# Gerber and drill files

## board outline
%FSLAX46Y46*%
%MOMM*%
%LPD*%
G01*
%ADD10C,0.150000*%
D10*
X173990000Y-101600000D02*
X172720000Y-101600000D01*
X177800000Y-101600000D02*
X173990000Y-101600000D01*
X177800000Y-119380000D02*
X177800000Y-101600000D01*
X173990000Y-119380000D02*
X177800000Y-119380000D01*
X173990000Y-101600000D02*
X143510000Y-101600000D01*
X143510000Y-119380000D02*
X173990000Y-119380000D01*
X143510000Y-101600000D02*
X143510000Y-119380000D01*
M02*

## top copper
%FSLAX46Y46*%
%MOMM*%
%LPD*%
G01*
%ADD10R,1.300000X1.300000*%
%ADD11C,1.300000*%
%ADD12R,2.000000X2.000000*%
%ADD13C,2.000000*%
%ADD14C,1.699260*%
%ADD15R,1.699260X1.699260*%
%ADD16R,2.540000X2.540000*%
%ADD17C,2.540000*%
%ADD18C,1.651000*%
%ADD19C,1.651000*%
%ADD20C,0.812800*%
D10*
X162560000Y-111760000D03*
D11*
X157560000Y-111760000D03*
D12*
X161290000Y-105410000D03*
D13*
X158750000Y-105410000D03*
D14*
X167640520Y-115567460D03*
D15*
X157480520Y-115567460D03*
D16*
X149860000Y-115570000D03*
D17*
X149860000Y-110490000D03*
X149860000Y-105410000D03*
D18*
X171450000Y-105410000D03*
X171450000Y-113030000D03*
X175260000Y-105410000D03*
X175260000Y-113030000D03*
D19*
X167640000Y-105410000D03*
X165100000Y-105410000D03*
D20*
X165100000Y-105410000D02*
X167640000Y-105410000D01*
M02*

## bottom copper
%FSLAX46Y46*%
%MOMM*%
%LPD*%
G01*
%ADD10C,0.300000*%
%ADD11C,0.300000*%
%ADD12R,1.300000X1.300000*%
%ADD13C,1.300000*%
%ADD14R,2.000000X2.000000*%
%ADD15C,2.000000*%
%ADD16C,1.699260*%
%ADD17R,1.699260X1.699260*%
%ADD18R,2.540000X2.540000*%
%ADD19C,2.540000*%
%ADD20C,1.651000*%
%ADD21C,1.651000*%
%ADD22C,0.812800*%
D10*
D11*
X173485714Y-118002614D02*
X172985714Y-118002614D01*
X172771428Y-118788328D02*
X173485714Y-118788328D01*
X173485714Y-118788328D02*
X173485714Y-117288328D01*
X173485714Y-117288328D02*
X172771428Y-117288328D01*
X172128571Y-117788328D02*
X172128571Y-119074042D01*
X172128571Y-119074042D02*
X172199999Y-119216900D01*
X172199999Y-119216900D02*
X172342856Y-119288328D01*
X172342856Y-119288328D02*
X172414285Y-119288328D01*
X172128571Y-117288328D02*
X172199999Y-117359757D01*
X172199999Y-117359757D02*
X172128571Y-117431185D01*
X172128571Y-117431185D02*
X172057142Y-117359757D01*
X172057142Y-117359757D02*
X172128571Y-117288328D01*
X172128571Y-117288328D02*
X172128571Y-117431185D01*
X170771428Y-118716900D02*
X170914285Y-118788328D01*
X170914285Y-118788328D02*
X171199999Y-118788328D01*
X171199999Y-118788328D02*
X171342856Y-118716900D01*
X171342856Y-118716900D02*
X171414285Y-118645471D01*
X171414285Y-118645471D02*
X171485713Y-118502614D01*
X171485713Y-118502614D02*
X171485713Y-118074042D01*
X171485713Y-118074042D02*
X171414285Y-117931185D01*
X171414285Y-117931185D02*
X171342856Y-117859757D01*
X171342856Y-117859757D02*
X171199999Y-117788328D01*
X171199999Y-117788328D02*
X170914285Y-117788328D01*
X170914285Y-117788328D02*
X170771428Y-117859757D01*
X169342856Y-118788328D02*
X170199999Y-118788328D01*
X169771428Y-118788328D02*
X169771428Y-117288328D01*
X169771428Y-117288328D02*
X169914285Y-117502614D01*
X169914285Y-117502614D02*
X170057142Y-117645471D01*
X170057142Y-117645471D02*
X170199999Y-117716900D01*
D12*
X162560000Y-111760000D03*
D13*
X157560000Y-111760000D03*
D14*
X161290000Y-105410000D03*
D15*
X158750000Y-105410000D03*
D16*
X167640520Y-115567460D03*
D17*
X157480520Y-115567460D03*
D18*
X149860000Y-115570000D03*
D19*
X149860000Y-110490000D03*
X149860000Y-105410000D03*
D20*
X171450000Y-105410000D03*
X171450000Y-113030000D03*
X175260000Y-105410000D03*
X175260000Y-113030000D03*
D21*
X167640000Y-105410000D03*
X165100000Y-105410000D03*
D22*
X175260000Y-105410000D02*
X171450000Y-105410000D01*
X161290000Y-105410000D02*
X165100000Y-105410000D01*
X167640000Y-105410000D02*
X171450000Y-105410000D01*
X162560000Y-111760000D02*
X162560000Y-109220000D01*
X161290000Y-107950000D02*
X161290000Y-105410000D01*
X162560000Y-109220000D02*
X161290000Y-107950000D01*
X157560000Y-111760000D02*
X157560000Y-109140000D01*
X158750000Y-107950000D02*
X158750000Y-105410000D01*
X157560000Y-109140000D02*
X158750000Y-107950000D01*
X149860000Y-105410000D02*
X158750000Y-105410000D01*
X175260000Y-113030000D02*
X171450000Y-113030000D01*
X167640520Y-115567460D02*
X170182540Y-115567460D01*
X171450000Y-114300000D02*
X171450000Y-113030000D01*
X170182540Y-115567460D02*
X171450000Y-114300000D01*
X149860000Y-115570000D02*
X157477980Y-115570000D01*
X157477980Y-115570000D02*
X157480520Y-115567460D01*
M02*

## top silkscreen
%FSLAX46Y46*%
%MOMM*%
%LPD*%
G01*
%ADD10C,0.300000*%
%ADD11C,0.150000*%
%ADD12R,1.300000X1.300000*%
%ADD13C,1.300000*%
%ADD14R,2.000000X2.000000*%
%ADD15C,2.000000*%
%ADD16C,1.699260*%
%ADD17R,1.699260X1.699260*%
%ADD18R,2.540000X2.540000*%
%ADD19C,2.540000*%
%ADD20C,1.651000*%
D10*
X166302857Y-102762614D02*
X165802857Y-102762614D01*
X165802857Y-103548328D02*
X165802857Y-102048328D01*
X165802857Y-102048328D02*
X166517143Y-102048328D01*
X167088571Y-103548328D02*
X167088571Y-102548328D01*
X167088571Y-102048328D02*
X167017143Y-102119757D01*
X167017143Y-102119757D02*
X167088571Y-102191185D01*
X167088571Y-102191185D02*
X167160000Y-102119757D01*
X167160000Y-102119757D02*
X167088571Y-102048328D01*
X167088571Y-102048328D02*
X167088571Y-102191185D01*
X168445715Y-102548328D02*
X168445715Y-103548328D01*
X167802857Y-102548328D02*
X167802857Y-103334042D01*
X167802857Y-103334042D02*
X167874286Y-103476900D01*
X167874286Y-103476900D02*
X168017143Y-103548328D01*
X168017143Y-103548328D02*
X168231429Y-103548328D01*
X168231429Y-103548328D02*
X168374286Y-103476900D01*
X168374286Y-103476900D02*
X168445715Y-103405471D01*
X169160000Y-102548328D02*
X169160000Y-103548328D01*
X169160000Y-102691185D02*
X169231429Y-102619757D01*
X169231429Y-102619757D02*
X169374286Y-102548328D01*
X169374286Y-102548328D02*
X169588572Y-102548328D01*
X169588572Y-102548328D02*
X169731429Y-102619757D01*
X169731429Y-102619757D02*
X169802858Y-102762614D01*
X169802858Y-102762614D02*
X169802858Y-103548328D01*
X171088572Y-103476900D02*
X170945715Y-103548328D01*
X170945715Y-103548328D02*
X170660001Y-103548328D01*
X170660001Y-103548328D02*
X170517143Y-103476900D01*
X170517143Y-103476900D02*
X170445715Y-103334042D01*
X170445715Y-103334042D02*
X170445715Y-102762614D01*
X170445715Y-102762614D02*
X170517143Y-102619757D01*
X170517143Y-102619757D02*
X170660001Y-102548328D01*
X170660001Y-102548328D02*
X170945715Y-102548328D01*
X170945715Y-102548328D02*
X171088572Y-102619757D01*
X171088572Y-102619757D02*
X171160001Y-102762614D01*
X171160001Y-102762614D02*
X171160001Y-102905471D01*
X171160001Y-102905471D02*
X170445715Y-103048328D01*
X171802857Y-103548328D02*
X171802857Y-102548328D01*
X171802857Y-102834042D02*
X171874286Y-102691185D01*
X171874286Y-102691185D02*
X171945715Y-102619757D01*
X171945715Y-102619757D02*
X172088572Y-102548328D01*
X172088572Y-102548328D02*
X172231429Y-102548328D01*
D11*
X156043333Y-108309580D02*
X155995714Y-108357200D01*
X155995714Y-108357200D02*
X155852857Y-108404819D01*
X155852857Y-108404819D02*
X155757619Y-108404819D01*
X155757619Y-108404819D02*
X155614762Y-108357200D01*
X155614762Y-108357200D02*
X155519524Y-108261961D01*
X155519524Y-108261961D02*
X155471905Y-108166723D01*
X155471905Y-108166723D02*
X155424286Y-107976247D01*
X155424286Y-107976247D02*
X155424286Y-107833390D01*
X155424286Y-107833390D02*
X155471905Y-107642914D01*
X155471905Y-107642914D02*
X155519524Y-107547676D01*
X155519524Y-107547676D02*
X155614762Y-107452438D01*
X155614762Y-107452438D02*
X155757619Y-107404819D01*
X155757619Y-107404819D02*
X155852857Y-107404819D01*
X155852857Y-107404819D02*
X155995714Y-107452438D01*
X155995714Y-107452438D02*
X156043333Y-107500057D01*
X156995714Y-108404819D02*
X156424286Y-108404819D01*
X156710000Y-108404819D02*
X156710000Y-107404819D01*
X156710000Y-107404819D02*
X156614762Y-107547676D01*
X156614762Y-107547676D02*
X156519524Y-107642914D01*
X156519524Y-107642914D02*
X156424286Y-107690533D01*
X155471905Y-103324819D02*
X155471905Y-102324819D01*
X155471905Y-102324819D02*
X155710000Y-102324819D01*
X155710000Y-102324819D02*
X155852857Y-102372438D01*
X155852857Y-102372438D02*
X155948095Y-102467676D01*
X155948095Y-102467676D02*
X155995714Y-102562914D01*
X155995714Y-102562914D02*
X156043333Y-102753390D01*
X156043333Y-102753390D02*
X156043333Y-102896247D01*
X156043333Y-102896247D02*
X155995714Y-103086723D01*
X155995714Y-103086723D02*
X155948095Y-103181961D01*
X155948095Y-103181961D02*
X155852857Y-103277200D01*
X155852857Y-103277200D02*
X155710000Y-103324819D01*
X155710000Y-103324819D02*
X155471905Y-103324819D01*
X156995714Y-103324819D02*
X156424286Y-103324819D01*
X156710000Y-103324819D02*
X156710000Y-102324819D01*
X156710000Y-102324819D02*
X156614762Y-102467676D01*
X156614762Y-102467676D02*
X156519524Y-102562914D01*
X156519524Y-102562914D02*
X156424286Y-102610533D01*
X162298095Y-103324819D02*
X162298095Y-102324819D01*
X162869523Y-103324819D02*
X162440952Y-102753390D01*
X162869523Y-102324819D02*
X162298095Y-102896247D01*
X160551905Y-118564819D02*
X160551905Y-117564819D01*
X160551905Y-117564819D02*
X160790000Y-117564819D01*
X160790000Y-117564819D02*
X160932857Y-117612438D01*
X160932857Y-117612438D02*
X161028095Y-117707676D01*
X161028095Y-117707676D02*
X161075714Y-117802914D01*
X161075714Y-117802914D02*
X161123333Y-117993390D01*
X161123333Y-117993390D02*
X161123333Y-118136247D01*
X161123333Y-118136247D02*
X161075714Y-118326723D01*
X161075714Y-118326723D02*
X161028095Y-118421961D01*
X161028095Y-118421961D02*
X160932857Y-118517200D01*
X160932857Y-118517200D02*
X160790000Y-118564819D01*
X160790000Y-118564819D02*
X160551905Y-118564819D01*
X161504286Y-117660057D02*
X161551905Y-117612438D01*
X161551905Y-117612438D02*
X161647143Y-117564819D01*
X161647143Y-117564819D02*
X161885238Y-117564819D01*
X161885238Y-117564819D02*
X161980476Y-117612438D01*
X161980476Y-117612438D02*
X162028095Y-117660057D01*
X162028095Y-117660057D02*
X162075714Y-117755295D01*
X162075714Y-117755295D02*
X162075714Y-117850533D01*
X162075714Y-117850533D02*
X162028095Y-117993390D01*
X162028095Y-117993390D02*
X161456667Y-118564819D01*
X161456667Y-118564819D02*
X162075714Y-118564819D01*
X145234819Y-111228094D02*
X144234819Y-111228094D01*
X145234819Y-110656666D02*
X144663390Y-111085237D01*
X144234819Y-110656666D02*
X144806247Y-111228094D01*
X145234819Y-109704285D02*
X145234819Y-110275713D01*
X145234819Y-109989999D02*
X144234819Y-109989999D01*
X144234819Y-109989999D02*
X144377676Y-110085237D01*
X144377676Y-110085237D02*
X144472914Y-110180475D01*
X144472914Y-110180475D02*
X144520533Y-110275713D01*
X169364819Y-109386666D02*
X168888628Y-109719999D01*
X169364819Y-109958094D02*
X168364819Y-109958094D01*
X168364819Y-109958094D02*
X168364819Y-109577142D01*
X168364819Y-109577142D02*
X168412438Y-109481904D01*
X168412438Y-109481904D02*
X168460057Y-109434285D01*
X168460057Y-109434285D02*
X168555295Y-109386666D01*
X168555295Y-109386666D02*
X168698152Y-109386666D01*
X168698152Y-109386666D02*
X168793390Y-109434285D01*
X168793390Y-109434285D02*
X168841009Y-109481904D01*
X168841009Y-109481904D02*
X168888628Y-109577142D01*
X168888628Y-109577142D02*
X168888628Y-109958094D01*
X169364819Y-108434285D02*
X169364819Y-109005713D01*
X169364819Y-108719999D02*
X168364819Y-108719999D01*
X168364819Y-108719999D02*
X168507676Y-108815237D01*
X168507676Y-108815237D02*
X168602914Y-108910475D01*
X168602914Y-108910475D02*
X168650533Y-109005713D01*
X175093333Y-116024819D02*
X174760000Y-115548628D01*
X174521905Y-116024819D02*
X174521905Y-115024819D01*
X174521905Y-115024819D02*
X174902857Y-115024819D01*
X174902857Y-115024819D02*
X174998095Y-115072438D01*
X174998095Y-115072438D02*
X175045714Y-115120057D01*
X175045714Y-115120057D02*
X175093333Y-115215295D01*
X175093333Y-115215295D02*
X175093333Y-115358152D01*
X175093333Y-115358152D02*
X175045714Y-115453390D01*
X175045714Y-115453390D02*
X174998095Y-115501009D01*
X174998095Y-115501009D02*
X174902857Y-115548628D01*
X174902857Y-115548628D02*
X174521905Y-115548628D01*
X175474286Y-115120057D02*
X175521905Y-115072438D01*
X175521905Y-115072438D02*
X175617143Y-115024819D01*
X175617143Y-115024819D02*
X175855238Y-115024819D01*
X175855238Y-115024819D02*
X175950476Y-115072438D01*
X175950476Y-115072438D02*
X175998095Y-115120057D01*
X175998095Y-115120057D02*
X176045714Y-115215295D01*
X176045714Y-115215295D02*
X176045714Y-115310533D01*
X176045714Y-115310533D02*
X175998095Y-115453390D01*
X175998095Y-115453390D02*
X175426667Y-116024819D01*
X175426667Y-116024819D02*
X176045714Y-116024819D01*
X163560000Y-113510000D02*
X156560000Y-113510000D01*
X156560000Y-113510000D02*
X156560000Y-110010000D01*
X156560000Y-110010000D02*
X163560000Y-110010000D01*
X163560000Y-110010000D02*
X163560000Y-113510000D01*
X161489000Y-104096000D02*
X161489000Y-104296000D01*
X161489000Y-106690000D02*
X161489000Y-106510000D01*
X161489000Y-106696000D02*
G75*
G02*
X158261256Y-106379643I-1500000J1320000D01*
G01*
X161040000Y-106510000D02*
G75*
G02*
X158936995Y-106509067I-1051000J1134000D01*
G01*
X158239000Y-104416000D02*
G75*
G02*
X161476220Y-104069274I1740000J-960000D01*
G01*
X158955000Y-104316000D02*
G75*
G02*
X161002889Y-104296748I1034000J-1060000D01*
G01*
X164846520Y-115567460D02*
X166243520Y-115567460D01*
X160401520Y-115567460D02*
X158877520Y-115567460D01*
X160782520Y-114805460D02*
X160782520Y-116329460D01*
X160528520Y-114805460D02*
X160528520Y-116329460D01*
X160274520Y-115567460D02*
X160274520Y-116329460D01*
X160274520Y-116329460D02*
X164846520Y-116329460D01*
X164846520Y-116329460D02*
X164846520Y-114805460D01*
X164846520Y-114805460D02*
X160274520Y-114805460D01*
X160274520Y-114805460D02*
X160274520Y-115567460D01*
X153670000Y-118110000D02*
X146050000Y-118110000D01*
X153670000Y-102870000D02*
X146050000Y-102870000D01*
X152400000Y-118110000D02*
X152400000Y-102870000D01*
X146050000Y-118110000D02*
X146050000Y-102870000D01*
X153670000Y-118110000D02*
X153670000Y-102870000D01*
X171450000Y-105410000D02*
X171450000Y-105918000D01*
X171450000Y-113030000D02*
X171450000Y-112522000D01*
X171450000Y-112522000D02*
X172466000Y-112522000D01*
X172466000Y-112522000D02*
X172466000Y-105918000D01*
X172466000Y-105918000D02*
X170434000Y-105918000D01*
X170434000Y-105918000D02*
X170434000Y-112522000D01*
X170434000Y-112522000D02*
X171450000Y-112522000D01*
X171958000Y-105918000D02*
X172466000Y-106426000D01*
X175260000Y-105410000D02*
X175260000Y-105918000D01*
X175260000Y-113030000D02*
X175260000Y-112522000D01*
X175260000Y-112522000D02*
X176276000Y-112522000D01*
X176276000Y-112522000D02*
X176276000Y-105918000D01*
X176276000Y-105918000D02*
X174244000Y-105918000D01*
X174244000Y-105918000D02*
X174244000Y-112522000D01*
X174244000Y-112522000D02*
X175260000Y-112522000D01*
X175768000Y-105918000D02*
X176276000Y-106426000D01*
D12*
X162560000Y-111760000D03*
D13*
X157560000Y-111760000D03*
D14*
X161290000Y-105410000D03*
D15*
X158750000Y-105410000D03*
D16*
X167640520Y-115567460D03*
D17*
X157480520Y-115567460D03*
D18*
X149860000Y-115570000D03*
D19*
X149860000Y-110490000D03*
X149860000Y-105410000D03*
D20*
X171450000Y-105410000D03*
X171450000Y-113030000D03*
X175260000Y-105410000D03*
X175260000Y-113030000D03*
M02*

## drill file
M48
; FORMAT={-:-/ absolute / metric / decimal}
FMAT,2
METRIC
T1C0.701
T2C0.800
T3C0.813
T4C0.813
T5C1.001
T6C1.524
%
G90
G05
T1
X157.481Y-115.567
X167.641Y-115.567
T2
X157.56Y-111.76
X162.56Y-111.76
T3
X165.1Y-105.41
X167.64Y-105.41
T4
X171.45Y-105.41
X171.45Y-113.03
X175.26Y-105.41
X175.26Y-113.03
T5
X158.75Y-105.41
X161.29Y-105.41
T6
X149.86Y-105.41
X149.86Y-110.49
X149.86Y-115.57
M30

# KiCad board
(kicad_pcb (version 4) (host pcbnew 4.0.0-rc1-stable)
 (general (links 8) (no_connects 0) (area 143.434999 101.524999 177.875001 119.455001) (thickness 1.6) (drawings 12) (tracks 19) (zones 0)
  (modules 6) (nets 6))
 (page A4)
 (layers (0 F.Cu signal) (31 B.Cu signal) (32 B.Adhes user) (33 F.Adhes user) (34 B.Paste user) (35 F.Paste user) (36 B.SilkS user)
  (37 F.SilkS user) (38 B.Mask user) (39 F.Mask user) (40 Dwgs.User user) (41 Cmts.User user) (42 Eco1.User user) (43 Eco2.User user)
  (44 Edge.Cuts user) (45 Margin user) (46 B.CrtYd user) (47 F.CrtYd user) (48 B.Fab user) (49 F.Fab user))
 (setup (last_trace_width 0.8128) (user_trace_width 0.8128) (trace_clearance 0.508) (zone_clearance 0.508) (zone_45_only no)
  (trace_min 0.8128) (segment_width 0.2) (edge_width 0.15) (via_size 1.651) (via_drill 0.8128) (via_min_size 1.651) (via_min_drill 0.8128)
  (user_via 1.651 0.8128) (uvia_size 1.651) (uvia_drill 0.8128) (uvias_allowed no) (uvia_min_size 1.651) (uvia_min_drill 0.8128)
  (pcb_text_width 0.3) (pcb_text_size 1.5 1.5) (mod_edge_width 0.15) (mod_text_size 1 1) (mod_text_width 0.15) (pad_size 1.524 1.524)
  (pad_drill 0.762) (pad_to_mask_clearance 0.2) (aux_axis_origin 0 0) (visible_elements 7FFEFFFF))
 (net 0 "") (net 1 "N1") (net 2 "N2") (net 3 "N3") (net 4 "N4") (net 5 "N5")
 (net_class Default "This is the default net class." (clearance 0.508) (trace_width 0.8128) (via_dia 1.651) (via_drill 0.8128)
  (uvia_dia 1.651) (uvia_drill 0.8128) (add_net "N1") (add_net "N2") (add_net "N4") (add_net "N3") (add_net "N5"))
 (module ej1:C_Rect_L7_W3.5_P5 (layer F.Cu) (at 162.56 111.76 180)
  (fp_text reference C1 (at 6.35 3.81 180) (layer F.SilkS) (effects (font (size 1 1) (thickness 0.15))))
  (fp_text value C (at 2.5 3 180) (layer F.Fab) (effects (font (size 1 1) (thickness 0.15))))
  (fp_line (start -1 -1.75) (end 6 -1.75) (layer F.SilkS) (width 0.15))
  (fp_line (start 6 -1.75) (end 6 1.75) (layer F.SilkS) (width 0.15))
  (fp_line (start 6 1.75) (end -1 1.75) (layer F.SilkS) (width 0.15))
  (fp_line (start -1 1.75) (end -1 -1.75) (layer F.SilkS) (width 0.15))
  (pad 1 thru_hole rect (at 0 0 180) (size 1.3 1.3) (drill 0.8) (layers *.Cu *.Mask F.SilkS) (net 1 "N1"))
  (pad 2 thru_hole circle (at 5 0 180) (size 1.3 1.3) (drill 0.8) (layers *.Cu *.Mask F.SilkS) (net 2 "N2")))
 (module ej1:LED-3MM (layer F.Cu) (at 161.29 105.41 180)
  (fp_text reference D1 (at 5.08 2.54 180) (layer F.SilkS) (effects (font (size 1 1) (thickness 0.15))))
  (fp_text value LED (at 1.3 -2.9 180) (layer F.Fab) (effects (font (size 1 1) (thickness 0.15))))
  (fp_line (start -0.199 1.314) (end -0.199 1.114) (layer F.SilkS) (width 0.15))
  (fp_line (start -0.199 -1.28) (end -0.199 -1.1) (layer F.SilkS) (width 0.15))
  (fp_arc (start 1.301 0.034) (end -0.199 -1.286) (angle 108.5) (layer F.SilkS) (width 0.15))
  (fp_arc (start 1.301 0.034) (end 0.25 -1.1) (angle 85.7) (layer F.SilkS) (width 0.15))
  (fp_arc (start 1.311 0.034) (end 3.051 0.994) (angle 110) (layer F.SilkS) (width 0.15))
  (fp_arc (start 1.301 0.034) (end 2.335 1.094) (angle 87.5) (layer F.SilkS) (width 0.15))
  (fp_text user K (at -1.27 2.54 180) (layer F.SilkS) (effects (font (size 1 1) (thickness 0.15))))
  (pad 1 thru_hole rect (at 0 0 270) (size 2 2) (drill 1.00076) (layers *.Cu *.Mask F.SilkS) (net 1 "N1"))
  (pad 2 thru_hole circle (at 2.54 0 180) (size 2 2) (drill 1.00076) (layers *.Cu *.Mask F.SilkS) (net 2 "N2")))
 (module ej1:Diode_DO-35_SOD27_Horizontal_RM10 (layer F.Cu) (at 157.48 115.57)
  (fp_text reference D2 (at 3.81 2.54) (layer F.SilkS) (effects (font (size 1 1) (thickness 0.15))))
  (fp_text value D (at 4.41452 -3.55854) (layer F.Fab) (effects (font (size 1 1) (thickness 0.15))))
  (fp_line (start 7.36652 -0.00254) (end 8.76352 -0.00254) (layer F.SilkS) (width 0.15))
  (fp_line (start 2.92152 -0.00254) (end 1.39752 -0.00254) (layer F.SilkS) (width 0.15))
  (fp_line (start 3.30252 -0.76454) (end 3.30252 0.75946) (layer F.SilkS) (width 0.15))
  (fp_line (start 3.04852 -0.76454) (end 3.04852 0.75946) (layer F.SilkS) (width 0.15))
  (fp_line (start 2.79452 -0.00254) (end 2.79452 0.75946) (layer F.SilkS) (width 0.15))
  (fp_line (start 2.79452 0.75946) (end 7.36652 0.75946) (layer F.SilkS) (width 0.15))
  (fp_line (start 7.36652 0.75946) (end 7.36652 -0.76454) (layer F.SilkS) (width 0.15))
  (fp_line (start 7.36652 -0.76454) (end 2.79452 -0.76454) (layer F.SilkS) (width 0.15))
  (fp_line (start 2.79452 -0.76454) (end 2.79452 -0.00254) (layer F.SilkS) (width 0.15))
  (pad 2 thru_hole circle (at 10.16052 -0.00254 180) (size 1.69926 1.69926) (drill 0.70104) (layers *.Cu *.Mask F.SilkS) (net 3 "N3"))
  (pad 1 thru_hole rect (at 0.00052 -0.00254 180) (size 1.69926 1.69926) (drill 0.70104) (layers *.Cu *.Mask F.SilkS) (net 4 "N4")))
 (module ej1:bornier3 (layer F.Cu) (at 149.86 110.49 90)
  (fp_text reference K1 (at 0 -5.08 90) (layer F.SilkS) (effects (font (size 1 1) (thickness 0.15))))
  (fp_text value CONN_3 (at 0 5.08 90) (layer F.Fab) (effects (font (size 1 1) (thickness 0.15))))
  (fp_line (start -7.62 3.81) (end -7.62 -3.81) (layer F.SilkS) (width 0.15))
  (fp_line (start 7.62 3.81) (end 7.62 -3.81) (layer F.SilkS) (width 0.15))
  (fp_line (start -7.62 2.54) (end 7.62 2.54) (layer F.SilkS) (width 0.15))
  (fp_line (start -7.62 -3.81) (end 7.62 -3.81) (layer F.SilkS) (width 0.15))
  (fp_line (start -7.62 3.81) (end 7.62 3.81) (layer F.SilkS) (width 0.15))
  (pad 1 thru_hole rect (at -5.08 0 90) (size 2.54 2.54) (drill 1.524) (layers *.Cu *.Mask F.SilkS) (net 4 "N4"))
  (pad 2 thru_hole circle (at 0 0 90) (size 2.54 2.54) (drill 1.524) (layers *.Cu *.Mask F.SilkS) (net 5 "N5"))
  (pad 3 thru_hole circle (at 5.08 0 90) (size 2.54 2.54) (drill 1.524) (layers *.Cu *.Mask F.SilkS) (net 2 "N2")))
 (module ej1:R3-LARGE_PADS (layer F.Cu) (at 171.45 109.22 270)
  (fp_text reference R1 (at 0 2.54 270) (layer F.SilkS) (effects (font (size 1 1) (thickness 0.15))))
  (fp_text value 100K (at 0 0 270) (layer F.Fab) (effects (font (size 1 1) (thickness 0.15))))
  (fp_line (start -3.81 0) (end -3.302 0) (layer F.SilkS) (width 0.15))
  (fp_line (start 3.81 0) (end 3.302 0) (layer F.SilkS) (width 0.15))
  (fp_line (start 3.302 0) (end 3.302 -1.016) (layer F.SilkS) (width 0.15))
  (fp_line (start 3.302 -1.016) (end -3.302 -1.016) (layer F.SilkS) (width 0.15))
  (fp_line (start -3.302 -1.016) (end -3.302 1.016) (layer F.SilkS) (width 0.15))
  (fp_line (start -3.302 1.016) (end 3.302 1.016) (layer F.SilkS) (width 0.15))
  (fp_line (start 3.302 1.016) (end 3.302 0) (layer F.SilkS) (width 0.15))
  (fp_line (start -3.302 -0.508) (end -2.794 -1.016) (layer F.SilkS) (width 0.15))
  (pad 1 thru_hole circle (at -3.81 0 270) (size 1.651 1.651) (drill 0.8128) (layers *.Cu *.Mask F.SilkS) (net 1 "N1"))
  (pad 2 thru_hole circle (at 3.81 0 270) (size 1.651 1.651) (drill 0.8128) (layers *.Cu *.Mask F.SilkS) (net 3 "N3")))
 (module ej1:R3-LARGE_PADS (layer F.Cu) (at 175.26 109.22 270)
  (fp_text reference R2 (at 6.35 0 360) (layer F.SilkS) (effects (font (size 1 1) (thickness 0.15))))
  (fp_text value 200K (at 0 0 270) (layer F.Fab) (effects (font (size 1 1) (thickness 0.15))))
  (fp_line (start -3.81 0) (end -3.302 0) (layer F.SilkS) (width 0.15))
  (fp_line (start 3.81 0) (end 3.302 0) (layer F.SilkS) (width 0.15))
  (fp_line (start 3.302 0) (end 3.302 -1.016) (layer F.SilkS) (width 0.15))
  (fp_line (start 3.302 -1.016) (end -3.302 -1.016) (layer F.SilkS) (width 0.15))
  (fp_line (start -3.302 -1.016) (end -3.302 1.016) (layer F.SilkS) (width 0.15))
  (fp_line (start -3.302 1.016) (end 3.302 1.016) (layer F.SilkS) (width 0.15))
  (fp_line (start 3.302 1.016) (end 3.302 0) (layer F.SilkS) (width 0.15))
  (fp_line (start -3.302 -0.508) (end -2.794 -1.016) (layer F.SilkS) (width 0.15))
  (pad 1 thru_hole circle (at -3.81 0 270) (size 1.651 1.651) (drill 0.8128) (layers *.Cu *.Mask F.SilkS) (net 1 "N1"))
  (pad 2 thru_hole circle (at 3.81 0 270) (size 1.651 1.651) (drill 0.8128) (layers *.Cu *.Mask F.SilkS) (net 3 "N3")))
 (gr_line (start 173.99 101.6) (end 172.72 101.6) (angle 90) (layer Edge.Cuts) (width 0.15))
 (gr_line (start 177.8 101.6) (end 173.99 101.6) (angle 90) (layer Edge.Cuts) (width 0.15))
 (gr_line (start 177.8 119.38) (end 177.8 101.6) (angle 90) (layer Edge.Cuts) (width 0.15))
 (gr_line (start 173.99 119.38) (end 177.8 119.38) (angle 90) (layer Edge.Cuts) (width 0.15))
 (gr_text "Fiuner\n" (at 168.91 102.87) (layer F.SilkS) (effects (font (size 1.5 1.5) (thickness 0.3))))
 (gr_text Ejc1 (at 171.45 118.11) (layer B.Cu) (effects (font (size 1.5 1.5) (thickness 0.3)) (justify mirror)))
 (gr_line (start 173.99 101.6) (end 143.51 101.6) (angle 90) (layer Edge.Cuts) (width 0.15))
 (gr_line (start 143.51 119.38) (end 173.99 119.38) (angle 90) (layer Edge.Cuts) (width 0.15))
 (gr_line (start 143.51 101.6) (end 143.51 119.38) (angle 90) (layer Edge.Cuts) (width 0.15))
 (segment (start 175.26 105.41) (end 171.45 105.41) (width 0.8128) (layer B.Cu) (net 1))
 (segment (start 161.29 105.41) (end 165.1 105.41) (width 0.8128) (layer B.Cu) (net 1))
 (segment (start 167.64 105.41) (end 171.45 105.41) (width 0.8128) (layer B.Cu) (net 1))
 (via (at 167.64 105.41) (size 1.651) (drill 0.8128) (layers F.Cu B.Cu) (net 1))
 (segment (start 165.1 105.41) (end 167.64 105.41) (width 0.8128) (layer F.Cu) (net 1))
 (via (at 165.1 105.41) (size 1.651) (drill 0.8128) (layers F.Cu B.Cu) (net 1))
 (segment (start 162.56 111.76) (end 162.56 109.22) (width 0.8128) (layer B.Cu) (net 1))
 (segment (start 161.29 107.95) (end 161.29 105.41) (width 0.8128) (layer B.Cu) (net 1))
 (segment (start 162.56 109.22) (end 161.29 107.95) (width 0.8128) (layer B.Cu) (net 1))
 (segment (start 157.56 111.76) (end 157.56 109.14) (width 0.8128) (layer B.Cu) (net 2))
 (segment (start 158.75 107.95) (end 158.75 105.41) (width 0.8128) (layer B.Cu) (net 2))
 (segment (start 157.56 109.14) (end 158.75 107.95) (width 0.8128) (layer B.Cu) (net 2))
 (segment (start 149.86 105.41) (end 158.75 105.41) (width 0.8128) (layer B.Cu) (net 2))
 (segment (start 175.26 113.03) (end 171.45 113.03) (width 0.8128) (layer B.Cu) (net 3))
 (segment (start 167.64052 115.56746) (end 170.18254 115.56746) (width 0.8128) (layer B.Cu) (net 3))
 (segment (start 171.45 114.3) (end 171.45 113.03) (width 0.8128) (layer B.Cu) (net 3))
 (segment (start 170.18254 115.56746) (end 171.45 114.3) (width 0.8128) (layer B.Cu) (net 3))
 (segment (start 149.86 115.57) (end 157.47798 115.57) (width 0.8128) (layer B.Cu) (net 4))
 (segment (start 157.47798 115.57) (end 157.48052 115.56746) (width 0.8128) (layer B.Cu) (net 4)))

